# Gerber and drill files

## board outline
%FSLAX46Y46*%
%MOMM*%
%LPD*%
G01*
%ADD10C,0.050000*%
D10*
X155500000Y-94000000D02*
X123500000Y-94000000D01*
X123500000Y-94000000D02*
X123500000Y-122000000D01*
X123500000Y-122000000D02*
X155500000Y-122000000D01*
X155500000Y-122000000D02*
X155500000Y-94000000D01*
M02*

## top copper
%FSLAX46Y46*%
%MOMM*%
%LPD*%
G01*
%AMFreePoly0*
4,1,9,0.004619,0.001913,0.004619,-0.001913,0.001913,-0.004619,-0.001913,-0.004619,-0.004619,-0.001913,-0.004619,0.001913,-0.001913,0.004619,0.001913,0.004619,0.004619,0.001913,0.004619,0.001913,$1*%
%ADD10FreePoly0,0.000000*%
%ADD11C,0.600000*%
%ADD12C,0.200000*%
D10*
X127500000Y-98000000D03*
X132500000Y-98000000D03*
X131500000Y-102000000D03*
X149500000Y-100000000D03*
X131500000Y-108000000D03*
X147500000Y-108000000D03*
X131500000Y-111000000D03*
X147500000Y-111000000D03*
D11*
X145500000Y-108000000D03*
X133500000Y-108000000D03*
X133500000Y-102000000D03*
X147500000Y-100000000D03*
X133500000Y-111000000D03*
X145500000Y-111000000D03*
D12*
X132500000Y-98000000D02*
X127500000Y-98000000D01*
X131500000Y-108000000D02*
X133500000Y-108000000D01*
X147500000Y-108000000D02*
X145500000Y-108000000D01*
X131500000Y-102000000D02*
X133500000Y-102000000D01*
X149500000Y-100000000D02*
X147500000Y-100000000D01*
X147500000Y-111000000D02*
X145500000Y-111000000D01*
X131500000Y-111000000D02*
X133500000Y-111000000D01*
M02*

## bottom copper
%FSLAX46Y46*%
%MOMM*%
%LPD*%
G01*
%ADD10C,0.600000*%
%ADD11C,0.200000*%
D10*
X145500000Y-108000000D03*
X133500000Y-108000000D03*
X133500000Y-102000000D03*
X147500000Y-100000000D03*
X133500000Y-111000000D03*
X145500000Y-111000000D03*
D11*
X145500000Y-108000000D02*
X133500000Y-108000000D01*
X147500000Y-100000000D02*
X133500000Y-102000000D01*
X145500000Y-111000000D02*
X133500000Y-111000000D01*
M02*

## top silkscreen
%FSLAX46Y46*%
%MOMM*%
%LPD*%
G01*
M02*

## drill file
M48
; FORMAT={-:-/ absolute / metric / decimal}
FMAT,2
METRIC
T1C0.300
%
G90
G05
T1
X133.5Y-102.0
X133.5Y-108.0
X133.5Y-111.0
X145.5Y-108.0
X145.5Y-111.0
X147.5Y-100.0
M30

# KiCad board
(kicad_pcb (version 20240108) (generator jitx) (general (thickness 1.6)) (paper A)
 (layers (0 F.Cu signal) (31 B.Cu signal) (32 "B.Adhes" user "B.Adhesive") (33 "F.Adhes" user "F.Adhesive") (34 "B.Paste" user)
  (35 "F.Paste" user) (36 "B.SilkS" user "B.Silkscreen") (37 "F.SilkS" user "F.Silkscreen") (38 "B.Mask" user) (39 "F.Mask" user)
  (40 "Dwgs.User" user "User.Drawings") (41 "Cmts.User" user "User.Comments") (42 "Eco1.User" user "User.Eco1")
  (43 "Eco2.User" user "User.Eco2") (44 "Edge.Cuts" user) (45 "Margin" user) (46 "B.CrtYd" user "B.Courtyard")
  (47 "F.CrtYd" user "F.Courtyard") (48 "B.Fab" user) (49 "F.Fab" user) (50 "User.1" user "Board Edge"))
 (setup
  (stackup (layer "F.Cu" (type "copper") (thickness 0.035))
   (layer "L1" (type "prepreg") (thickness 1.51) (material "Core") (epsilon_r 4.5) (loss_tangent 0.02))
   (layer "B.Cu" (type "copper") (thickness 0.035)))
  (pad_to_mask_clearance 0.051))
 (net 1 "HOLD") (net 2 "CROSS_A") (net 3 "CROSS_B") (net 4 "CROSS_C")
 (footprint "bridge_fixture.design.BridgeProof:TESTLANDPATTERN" (layer F.Cu) (at 127.5 98.0 0.0)
  (pad p smd custom (at 0.0 0.0 0.0) (size 0.01 0.01) (options (clearance outline) (anchor circle)) (primitives) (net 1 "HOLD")
   (layers F.Cu))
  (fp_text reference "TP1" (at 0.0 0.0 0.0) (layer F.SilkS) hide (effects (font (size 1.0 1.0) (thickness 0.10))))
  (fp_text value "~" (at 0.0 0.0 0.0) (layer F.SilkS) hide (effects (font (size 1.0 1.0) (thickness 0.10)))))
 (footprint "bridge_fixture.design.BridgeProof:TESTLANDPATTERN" (layer F.Cu) (at 132.5 98.0 0.0)
  (pad p smd custom (at 0.0 0.0 0.0) (size 0.01 0.01) (options (clearance outline) (anchor circle)) (primitives) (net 1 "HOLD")
   (layers F.Cu))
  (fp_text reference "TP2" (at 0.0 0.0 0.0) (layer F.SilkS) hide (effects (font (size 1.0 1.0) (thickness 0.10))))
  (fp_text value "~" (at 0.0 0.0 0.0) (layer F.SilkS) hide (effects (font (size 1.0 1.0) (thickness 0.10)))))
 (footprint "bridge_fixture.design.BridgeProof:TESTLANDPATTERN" (layer F.Cu) (at 131.5 102.0 0.0)
  (pad p smd custom (at 0.0 0.0 0.0) (size 0.01 0.01) (options (clearance outline) (anchor circle)) (primitives) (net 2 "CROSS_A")
   (layers F.Cu))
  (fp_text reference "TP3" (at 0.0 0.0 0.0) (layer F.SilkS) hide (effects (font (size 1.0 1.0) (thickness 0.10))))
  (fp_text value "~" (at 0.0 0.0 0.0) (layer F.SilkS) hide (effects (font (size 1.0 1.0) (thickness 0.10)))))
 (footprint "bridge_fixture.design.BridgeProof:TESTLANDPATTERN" (layer F.Cu) (at 149.5 100.0 0.0)
  (pad p smd custom (at 0.0 0.0 0.0) (size 0.01 0.01) (options (clearance outline) (anchor circle)) (primitives) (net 2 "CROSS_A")
   (layers F.Cu))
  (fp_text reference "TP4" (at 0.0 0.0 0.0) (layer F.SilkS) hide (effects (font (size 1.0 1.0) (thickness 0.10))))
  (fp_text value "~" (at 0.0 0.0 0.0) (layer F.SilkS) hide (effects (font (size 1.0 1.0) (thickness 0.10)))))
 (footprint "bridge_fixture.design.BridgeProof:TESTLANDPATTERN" (layer F.Cu) (at 131.5 108.0 0.0)
  (pad p smd custom (at 0.0 0.0 0.0) (size 0.01 0.01) (options (clearance outline) (anchor circle)) (primitives) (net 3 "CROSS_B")
   (layers F.Cu))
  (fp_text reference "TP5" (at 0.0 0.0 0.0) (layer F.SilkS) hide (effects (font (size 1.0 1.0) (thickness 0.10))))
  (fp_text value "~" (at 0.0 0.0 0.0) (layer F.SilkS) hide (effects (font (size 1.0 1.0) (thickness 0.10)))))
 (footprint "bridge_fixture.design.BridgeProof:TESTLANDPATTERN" (layer F.Cu) (at 147.5 108.0 0.0)
  (pad p smd custom (at 0.0 0.0 0.0) (size 0.01 0.01) (options (clearance outline) (anchor circle)) (primitives) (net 3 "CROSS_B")
   (layers F.Cu))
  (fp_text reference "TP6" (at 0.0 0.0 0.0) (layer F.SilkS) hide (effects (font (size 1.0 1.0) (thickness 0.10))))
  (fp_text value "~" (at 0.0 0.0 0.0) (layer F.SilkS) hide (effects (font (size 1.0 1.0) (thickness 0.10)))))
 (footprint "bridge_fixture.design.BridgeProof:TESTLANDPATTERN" (layer F.Cu) (at 131.5 111.0 0.0)
  (pad p smd custom (at 0.0 0.0 0.0) (size 0.01 0.01) (options (clearance outline) (anchor circle)) (primitives) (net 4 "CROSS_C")
   (layers F.Cu))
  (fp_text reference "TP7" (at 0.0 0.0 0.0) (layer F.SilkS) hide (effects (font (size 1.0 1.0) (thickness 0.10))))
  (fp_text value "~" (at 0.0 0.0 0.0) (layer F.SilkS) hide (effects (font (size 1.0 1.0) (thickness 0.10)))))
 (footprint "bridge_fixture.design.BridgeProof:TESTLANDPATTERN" (layer F.Cu) (at 147.5 111.0 0.0)
  (pad p smd custom (at 0.0 0.0 0.0) (size 0.01 0.01) (options (clearance outline) (anchor circle)) (primitives) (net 4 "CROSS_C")
   (layers F.Cu))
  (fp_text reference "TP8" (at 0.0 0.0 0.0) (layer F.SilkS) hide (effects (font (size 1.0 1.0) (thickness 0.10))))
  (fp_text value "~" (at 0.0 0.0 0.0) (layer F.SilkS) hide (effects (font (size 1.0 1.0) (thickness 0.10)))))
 (segment (start 132.5 98.0) (end 127.5 98.0) (layer F.Cu) (width 0.2) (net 1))
 (segment (start 145.500000001462 108.000000001315) (end 133.499999998538 108.000000001315) (layer B.Cu) (width 0.2) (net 3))
 (segment (start 131.5 108.0) (end 133.499999998538 108.000000001315) (layer F.Cu) (width 0.2) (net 3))
 (segment (start 147.5 108.0) (end 145.500000001462 108.000000001315) (layer F.Cu) (width 0.2) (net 3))
 (segment (start 147.500000004939 99.9999999974389) (end 133.499999995061 101.999999997439) (layer B.Cu) (width 0.2) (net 2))
 (segment (start 131.5 102.0) (end 133.499999995061 101.999999997439) (layer F.Cu) (width 0.2) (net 2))
 (segment (start 149.5 100.0) (end 147.500000004939 99.9999999974389) (layer F.Cu) (width 0.2) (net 2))
 (segment (start 145.500000001462 110.999999998685) (end 133.499999998538 110.999999998685) (layer B.Cu) (width 0.2) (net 4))
 (segment (start 147.5 111.0) (end 145.500000001462 110.999999998685) (layer F.Cu) (width 0.2) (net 4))
 (segment (start 131.5 111.0) (end 133.499999998538 110.999999998685) (layer F.Cu) (width 0.2) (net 4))
 (via (at 145.500000001462 108.000000001315) (size 0.6) (drill 0.3) (layers F.Cu B.Cu) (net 3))
 (via (at 133.499999998538 108.000000001315) (size 0.6) (drill 0.3) (layers F.Cu B.Cu) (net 3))
 (via (at 133.499999995061 101.999999997439) (size 0.6) (drill 0.3) (layers F.Cu B.Cu) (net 2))
 (via (at 147.500000004939 99.9999999974389) (size 0.6) (drill 0.3) (layers F.Cu B.Cu) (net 2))
 (via (at 133.499999998538 110.999999998685) (size 0.6) (drill 0.3) (layers F.Cu B.Cu) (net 4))
 (via (at 145.500000001462 110.999999998685) (size 0.6) (drill 0.3) (layers F.Cu B.Cu) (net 4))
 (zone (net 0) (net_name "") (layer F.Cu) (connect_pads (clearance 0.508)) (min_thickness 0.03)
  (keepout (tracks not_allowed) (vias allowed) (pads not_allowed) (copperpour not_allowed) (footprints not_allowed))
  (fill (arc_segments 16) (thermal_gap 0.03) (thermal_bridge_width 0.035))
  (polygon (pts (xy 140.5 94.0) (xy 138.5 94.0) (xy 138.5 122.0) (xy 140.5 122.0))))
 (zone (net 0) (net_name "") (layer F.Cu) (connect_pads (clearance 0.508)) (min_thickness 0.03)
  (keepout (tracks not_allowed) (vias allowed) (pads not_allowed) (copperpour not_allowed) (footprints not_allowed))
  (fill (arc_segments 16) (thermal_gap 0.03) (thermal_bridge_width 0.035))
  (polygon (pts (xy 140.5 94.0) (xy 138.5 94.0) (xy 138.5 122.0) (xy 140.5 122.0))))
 (gr_line (start 155.5 94.0) (end 123.5 94.0) (layer Edge.Cuts) (stroke (width 0.05) (type solid)))
 (gr_line (start 123.5 94.0) (end 123.5 122.0) (layer Edge.Cuts) (stroke (width 0.05) (type solid)))
 (gr_line (start 123.5 122.0) (end 155.5 122.0) (layer Edge.Cuts) (stroke (width 0.05) (type solid)))
 (gr_line (start 155.5 122.0) (end 155.5 94.0) (layer Edge.Cuts) (stroke (width 0.05) (type solid)))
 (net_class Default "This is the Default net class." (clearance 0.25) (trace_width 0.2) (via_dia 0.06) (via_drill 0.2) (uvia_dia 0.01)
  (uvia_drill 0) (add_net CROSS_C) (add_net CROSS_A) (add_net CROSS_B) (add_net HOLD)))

